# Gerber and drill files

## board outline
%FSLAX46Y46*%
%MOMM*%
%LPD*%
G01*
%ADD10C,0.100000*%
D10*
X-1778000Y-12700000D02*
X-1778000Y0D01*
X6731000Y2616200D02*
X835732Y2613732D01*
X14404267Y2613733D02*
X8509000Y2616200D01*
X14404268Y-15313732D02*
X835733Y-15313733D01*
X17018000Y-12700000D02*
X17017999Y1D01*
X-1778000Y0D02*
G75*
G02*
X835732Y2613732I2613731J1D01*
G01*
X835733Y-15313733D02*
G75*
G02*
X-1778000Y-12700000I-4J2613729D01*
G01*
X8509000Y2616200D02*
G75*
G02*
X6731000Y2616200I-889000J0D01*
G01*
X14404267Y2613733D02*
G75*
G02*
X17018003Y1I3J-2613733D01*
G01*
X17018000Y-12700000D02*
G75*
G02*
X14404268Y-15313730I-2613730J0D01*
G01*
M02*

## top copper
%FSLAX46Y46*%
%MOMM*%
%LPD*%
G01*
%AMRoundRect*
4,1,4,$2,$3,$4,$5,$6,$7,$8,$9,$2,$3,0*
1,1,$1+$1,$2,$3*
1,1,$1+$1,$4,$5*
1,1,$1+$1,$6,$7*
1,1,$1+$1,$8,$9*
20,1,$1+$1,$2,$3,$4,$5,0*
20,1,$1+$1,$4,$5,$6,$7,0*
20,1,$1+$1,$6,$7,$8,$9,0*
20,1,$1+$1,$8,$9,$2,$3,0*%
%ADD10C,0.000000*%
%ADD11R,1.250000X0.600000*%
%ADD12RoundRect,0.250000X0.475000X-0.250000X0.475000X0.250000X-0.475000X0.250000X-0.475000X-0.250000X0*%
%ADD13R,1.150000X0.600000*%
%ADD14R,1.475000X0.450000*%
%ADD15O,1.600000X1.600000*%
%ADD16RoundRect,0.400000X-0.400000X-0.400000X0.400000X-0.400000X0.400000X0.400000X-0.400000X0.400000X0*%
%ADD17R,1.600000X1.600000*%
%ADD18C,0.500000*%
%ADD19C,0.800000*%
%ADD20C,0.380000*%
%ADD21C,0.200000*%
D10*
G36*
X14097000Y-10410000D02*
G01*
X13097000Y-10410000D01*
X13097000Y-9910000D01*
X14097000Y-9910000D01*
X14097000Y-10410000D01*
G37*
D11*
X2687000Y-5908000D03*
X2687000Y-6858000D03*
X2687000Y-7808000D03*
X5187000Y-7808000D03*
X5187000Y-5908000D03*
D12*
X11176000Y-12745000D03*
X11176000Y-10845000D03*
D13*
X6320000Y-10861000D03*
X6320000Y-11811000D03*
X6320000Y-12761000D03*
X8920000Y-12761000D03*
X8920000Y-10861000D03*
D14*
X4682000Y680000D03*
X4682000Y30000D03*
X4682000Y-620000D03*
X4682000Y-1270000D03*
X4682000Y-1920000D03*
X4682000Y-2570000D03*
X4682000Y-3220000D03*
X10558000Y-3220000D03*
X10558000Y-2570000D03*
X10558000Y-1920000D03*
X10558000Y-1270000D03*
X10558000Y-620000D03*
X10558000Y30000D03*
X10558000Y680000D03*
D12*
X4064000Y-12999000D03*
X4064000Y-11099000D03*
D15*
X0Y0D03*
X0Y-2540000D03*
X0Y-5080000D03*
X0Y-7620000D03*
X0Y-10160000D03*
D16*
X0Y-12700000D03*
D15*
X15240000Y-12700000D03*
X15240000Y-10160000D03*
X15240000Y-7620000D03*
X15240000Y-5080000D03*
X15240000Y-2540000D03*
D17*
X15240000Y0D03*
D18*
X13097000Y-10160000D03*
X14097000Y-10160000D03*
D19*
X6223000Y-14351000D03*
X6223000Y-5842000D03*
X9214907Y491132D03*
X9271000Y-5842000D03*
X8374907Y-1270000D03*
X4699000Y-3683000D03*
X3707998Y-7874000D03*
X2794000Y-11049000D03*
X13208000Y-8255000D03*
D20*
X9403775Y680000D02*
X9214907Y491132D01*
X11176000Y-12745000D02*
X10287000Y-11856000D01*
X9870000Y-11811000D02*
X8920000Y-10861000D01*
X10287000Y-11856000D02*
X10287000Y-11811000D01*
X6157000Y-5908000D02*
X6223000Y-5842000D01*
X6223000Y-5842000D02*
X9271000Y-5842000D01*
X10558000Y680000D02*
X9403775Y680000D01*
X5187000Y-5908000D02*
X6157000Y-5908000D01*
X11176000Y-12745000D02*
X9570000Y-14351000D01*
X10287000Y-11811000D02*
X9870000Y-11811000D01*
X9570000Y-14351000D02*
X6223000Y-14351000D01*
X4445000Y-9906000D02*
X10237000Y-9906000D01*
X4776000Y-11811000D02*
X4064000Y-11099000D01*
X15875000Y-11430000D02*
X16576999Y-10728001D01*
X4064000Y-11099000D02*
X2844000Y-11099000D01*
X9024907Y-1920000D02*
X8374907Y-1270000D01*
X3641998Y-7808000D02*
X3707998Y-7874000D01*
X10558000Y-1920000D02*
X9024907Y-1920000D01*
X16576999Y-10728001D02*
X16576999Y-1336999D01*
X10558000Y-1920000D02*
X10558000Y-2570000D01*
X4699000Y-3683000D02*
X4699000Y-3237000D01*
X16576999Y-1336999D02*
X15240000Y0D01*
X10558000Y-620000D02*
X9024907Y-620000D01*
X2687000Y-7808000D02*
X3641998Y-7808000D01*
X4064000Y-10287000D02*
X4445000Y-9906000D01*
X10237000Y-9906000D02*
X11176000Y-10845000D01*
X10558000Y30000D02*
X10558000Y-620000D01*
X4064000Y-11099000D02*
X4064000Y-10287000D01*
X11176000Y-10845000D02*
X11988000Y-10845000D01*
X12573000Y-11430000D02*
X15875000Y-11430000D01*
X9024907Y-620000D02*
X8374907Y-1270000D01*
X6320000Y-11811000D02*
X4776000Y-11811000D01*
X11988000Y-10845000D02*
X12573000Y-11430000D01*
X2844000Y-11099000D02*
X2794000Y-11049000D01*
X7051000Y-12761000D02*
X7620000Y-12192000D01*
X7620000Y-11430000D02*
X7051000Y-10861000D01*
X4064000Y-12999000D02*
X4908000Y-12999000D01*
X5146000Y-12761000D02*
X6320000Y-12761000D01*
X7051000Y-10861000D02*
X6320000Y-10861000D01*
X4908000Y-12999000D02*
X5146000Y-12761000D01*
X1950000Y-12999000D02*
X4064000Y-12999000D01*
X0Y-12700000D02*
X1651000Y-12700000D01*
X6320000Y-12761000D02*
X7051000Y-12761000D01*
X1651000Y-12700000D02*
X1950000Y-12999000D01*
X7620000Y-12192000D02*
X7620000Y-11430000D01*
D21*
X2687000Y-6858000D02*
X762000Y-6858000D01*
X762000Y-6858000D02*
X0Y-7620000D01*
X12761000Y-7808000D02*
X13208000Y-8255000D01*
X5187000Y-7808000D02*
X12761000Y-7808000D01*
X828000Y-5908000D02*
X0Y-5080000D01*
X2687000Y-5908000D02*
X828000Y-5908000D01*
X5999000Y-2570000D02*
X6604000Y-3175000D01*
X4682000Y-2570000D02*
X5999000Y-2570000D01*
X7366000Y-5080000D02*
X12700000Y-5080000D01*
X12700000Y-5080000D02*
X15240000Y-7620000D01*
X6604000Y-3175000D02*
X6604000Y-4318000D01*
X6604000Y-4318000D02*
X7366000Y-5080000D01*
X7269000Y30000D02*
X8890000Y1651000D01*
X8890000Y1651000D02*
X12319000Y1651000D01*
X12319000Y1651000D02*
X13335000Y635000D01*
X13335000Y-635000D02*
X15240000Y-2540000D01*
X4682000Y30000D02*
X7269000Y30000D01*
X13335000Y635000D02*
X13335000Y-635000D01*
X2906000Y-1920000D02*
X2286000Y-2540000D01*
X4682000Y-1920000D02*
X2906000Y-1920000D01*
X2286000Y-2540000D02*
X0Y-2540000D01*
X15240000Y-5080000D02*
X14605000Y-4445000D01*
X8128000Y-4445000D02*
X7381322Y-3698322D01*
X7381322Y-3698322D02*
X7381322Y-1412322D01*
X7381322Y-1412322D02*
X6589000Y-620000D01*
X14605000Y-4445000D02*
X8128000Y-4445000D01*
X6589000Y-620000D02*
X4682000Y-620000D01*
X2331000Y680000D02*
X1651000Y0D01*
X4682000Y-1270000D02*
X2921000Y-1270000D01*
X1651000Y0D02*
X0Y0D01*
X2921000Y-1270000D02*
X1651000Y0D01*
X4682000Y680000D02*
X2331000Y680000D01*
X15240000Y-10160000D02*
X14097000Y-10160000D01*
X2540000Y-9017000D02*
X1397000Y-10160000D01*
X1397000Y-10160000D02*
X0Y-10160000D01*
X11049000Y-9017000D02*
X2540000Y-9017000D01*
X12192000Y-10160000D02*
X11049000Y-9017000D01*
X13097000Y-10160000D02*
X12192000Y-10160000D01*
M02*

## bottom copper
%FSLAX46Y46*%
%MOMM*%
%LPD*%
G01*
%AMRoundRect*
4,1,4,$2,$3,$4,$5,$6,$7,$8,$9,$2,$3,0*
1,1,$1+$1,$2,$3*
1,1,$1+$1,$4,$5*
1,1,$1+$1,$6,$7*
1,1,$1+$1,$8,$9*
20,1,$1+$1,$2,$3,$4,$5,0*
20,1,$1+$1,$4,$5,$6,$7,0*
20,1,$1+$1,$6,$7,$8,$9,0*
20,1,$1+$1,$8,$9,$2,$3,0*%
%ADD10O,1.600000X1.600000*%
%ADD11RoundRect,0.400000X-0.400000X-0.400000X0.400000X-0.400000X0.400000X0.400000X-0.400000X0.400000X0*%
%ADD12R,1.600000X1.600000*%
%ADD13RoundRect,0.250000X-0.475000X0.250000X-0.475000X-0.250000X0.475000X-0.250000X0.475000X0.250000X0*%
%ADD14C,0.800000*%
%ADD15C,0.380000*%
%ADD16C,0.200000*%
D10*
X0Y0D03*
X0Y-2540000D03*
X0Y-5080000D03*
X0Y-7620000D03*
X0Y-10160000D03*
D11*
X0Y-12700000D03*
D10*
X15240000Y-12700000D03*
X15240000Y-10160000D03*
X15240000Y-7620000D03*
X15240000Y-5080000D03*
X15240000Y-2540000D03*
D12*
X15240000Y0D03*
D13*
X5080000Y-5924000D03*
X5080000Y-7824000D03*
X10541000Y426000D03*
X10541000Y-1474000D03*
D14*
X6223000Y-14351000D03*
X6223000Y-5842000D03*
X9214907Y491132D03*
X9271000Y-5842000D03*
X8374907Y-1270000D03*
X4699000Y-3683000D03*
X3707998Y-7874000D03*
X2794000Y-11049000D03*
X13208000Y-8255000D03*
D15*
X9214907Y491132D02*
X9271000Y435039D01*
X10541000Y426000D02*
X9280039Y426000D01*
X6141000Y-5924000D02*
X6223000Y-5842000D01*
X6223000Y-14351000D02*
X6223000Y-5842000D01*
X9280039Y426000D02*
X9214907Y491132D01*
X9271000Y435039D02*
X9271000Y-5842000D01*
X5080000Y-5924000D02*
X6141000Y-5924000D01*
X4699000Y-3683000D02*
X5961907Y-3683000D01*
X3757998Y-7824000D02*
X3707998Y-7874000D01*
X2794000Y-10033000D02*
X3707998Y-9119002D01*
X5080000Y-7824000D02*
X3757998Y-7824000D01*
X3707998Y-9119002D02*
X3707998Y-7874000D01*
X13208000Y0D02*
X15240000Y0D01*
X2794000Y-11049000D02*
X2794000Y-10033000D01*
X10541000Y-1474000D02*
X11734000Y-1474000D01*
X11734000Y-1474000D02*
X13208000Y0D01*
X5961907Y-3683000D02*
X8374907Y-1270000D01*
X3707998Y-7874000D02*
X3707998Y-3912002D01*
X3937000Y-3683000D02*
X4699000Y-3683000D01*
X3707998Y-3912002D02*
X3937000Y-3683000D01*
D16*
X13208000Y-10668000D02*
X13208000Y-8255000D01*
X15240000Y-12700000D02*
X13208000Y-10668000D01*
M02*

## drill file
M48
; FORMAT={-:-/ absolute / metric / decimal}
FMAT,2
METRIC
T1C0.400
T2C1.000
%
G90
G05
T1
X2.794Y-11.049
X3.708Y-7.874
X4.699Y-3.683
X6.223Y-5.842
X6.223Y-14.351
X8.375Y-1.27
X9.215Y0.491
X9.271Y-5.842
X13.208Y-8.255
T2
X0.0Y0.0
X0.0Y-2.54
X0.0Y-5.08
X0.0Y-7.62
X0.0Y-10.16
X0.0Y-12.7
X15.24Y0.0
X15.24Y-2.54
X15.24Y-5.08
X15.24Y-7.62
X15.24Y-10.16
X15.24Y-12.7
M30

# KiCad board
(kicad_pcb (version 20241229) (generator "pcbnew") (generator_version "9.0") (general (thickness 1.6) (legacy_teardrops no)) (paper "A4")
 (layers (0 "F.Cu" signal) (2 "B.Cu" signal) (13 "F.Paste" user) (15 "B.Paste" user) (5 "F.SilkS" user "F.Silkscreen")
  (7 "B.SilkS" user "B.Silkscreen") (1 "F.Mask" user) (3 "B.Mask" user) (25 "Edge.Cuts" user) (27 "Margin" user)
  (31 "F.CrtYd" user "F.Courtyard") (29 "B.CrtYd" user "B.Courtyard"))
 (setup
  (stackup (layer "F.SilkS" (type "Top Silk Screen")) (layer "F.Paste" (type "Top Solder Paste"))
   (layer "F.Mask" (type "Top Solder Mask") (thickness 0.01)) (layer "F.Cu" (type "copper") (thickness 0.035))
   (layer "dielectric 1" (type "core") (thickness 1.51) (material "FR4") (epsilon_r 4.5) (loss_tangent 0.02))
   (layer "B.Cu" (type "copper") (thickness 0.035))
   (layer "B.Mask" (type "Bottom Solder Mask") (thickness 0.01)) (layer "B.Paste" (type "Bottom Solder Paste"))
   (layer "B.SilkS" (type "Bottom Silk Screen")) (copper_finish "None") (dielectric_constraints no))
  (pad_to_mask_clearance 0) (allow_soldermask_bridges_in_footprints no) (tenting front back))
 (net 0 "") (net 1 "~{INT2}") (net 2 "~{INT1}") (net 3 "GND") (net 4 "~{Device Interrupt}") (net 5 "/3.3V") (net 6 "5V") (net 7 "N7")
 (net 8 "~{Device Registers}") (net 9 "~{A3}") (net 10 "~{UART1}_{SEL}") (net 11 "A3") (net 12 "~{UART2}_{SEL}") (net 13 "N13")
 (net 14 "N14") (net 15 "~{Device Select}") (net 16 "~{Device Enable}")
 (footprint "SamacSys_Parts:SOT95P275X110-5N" (layer "F.Cu") (at 3.937 6.858)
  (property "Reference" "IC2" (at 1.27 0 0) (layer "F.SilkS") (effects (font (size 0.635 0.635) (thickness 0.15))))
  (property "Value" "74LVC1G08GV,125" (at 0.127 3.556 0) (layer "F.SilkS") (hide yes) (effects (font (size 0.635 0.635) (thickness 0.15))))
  (pad "1" smd rect (at -1.25 -0.95 90) (size 0.6 1.25) (layers "F.Cu" "F.Mask" "F.Paste") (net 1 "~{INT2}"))
  (pad "2" smd rect (at -1.25 0 90) (size 0.6 1.25) (layers "F.Cu" "F.Mask" "F.Paste") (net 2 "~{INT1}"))
  (pad "3" smd rect (at -1.25 0.95 90) (size 0.6 1.25) (layers "F.Cu" "F.Mask" "F.Paste") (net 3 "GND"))
  (pad "4" smd rect (at 1.25 0.95 90) (size 0.6 1.25) (layers "F.Cu" "F.Mask" "F.Paste") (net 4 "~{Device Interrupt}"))
  (pad "5" smd rect (at 1.25 -0.95 90) (size 0.6 1.25) (layers "F.Cu" "F.Mask" "F.Paste") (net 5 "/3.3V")))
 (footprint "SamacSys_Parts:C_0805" (layer "F.Cu") (at 11.176 11.811)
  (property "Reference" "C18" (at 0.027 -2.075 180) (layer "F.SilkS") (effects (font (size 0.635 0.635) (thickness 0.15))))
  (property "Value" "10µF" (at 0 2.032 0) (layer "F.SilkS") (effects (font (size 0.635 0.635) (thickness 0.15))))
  (pad "1" smd roundrect (at 0 0.934 90) (size 1 1.45) (layers "F.Cu" "F.Mask" "F.Paste") (roundrect_rratio 0.25) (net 5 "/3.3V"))
  (pad "2" smd roundrect (at 0 -0.966 90) (size 1 1.45) (layers "F.Cu" "F.Mask" "F.Paste") (roundrect_rratio 0.25) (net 3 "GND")))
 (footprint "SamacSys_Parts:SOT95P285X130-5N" (layer "F.Cu") (at 7.62 11.811)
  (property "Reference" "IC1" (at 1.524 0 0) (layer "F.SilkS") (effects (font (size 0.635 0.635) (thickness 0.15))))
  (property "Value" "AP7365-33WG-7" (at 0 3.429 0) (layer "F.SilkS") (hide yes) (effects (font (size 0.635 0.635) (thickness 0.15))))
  (pad "1" smd rect (at -1.3 -0.95 90) (size 0.6 1.15) (layers "F.Cu" "F.Mask" "F.Paste") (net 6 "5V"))
  (pad "2" smd rect (at -1.3 0 90) (size 0.6 1.15) (layers "F.Cu" "F.Mask" "F.Paste") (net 3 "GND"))
  (pad "3" smd rect (at -1.3 0.95 90) (size 0.6 1.15) (layers "F.Cu" "F.Mask" "F.Paste") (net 6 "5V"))
  (pad "4" smd rect (at 1.3 0.95 90) (size 0.6 1.15) (layers "F.Cu" "F.Mask" "F.Paste") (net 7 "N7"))
  (pad "5" smd rect (at 1.3 -0.95 90) (size 0.6 1.15) (layers "F.Cu" "F.Mask" "F.Paste") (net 5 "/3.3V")))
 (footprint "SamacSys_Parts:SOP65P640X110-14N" (layer "F.Cu") (at 7.62 1.27)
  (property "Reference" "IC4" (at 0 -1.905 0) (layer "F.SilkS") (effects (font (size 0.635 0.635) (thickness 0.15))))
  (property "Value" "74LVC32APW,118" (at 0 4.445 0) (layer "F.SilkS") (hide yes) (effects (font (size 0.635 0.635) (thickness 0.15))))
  (pad "1" smd rect (at -2.938 -1.95 90) (size 0.45 1.475) (layers "F.Cu" "F.Mask" "F.Paste") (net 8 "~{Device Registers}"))
  (pad "2" smd rect (at -2.938 -1.3 90) (size 0.45 1.475) (layers "F.Cu" "F.Mask" "F.Paste") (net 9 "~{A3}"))
  (pad "3" smd rect (at -2.938 -0.65 90) (size 0.45 1.475) (layers "F.Cu" "F.Mask" "F.Paste") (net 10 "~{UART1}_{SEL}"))
  (pad "4" smd rect (at -2.938 0 90) (size 0.45 1.475) (layers "F.Cu" "F.Mask" "F.Paste") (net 8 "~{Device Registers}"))
  (pad "5" smd rect (at -2.938 0.65 90) (size 0.45 1.475) (layers "F.Cu" "F.Mask" "F.Paste") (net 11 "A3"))
  (pad "6" smd rect (at -2.938 1.3 90) (size 0.45 1.475) (layers "F.Cu" "F.Mask" "F.Paste") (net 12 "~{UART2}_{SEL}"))
  (pad "7" smd rect (at -2.938 1.95 90) (size 0.45 1.475) (layers "F.Cu" "F.Mask" "F.Paste") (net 3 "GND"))
  (pad "8" smd rect (at 2.938 1.95 90) (size 0.45 1.475) (layers "F.Cu" "F.Mask" "F.Paste") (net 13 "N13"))
  (pad "9" smd rect (at 2.938 1.3 90) (size 0.45 1.475) (layers "F.Cu" "F.Mask" "F.Paste") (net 3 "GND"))
  (pad "10" smd rect (at 2.938 0.65 90) (size 0.45 1.475) (layers "F.Cu" "F.Mask" "F.Paste") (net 3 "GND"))
  (pad "11" smd rect (at 2.938 0 90) (size 0.45 1.475) (layers "F.Cu" "F.Mask" "F.Paste") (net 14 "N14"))
  (pad "12" smd rect (at 2.938 -0.65 90) (size 0.45 1.475) (layers "F.Cu" "F.Mask" "F.Paste") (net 3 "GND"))
  (pad "13" smd rect (at 2.938 -1.3 90) (size 0.45 1.475) (layers "F.Cu" "F.Mask" "F.Paste") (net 3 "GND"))
  (pad "14" smd rect (at 2.938 -1.95 90) (size 0.45 1.475) (layers "F.Cu" "F.Mask" "F.Paste") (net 5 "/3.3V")))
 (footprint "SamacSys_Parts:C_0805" (layer "F.Cu") (at 4.064 12.065)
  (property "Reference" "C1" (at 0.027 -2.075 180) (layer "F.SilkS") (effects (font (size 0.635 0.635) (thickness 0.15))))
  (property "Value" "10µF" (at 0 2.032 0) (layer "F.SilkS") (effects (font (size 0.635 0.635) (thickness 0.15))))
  (pad "1" smd roundrect (at 0 0.934 90) (size 1 1.45) (layers "F.Cu" "F.Mask" "F.Paste") (roundrect_rratio 0.25) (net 6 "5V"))
  (pad "2" smd roundrect (at 0 -0.966 90) (size 1 1.45) (layers "F.Cu" "F.Mask" "F.Paste") (roundrect_rratio 0.25) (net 3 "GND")))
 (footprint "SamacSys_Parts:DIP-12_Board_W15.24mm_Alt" (layer "F.Cu") (at 0 0)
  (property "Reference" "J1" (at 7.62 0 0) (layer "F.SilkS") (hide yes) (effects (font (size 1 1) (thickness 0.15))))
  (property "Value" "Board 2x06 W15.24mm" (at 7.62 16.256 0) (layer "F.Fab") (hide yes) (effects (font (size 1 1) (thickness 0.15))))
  (fp_line (start -1.778 12.7) (end -1.778 0) (stroke (width 0.1) (type solid)) (layer "Edge.Cuts"))
  (fp_line (start 6.731 -2.6162) (end 0.835732 -2.613732) (stroke (width 0.1) (type solid)) (layer "Edge.Cuts"))
  (fp_line (start 14.404267 -2.613733) (end 8.509 -2.6162) (stroke (width 0.1) (type solid)) (layer "Edge.Cuts"))
  (fp_line (start 14.404268 15.313732) (end 0.835733 15.313733) (stroke (width 0.1) (type solid)) (layer "Edge.Cuts"))
  (fp_line (start 17.018 12.7) (end 17.017999 -0.000001) (stroke (width 0.1) (type solid)) (layer "Edge.Cuts"))
  (fp_arc (start -1.778 0) (mid -1.012456 -1.848188) (end 0.835732 -2.613732) (stroke (width 0.1) (type solid)) (layer "Edge.Cuts"))
  (fp_arc (start 0.835733 15.313733) (mid -1.012457 14.548189) (end -1.778 12.7) (stroke (width 0.1) (type solid)) (layer "Edge.Cuts"))
  (fp_arc (start 8.509 -2.6162) (mid 7.62 -1.7272) (end 6.731 -2.6162) (stroke (width 0.1) (type default)) (layer "Edge.Cuts"))
  (fp_arc (start 14.404267 -2.613733) (mid 16.252455 -1.848189) (end 17.017999 -0.000001) (stroke (width 0.1) (type solid))
   (layer "Edge.Cuts"))
  (fp_arc (start 17.018 12.7) (mid 16.252456 14.548187) (end 14.404268 15.313732) (stroke (width 0.1) (type solid)) (layer "Edge.Cuts"))
  (pad "1" thru_hole oval (at 0 0 180) (size 1.6 1.6) (drill 1) (layers "*.Cu" "*.Mask") (remove_unused_layers no)
   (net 8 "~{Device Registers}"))
  (pad "2" thru_hole oval (at 0 2.54) (size 1.6 1.6) (drill 1) (layers "*.Cu" "*.Mask") (remove_unused_layers no) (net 11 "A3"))
  (pad "3" thru_hole oval (at 0 5.08) (size 1.6 1.6) (drill 1) (layers "*.Cu" "*.Mask") (remove_unused_layers no) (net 1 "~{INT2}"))
  (pad "4" thru_hole oval (at 0 7.62 180) (size 1.6 1.6) (drill 1) (layers "*.Cu" "*.Mask") (remove_unused_layers no) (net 2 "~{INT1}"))
  (pad "5" thru_hole oval (at 0 10.16) (size 1.6 1.6) (drill 1) (layers "*.Cu" "*.Mask") (remove_unused_layers no)
   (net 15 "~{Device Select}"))
  (pad "6" thru_hole roundrect (at 0 12.7) (size 1.6 1.6) (drill 1) (layers "*.Cu" "*.Mask") (remove_unused_layers no)
   (roundrect_rratio 0.25) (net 6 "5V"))
  (pad "7" thru_hole oval (at 15.24 12.7 180) (size 1.6 1.6) (drill 1) (layers "*.Cu" "*.Mask") (remove_unused_layers no)
   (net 4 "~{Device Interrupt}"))
  (pad "8" thru_hole oval (at 15.24 10.16 180) (size 1.6 1.6) (drill 1) (layers "*.Cu" "*.Mask") (remove_unused_layers no)
   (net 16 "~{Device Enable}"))
  (pad "9" thru_hole oval (at 15.24 7.62 180) (size 1.6 1.6) (drill 1) (layers "*.Cu" "*.Mask") (remove_unused_layers no)
   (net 12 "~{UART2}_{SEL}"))
  (pad "10" thru_hole oval (at 15.24 5.08) (size 1.6 1.6) (drill 1) (layers "*.Cu" "*.Mask") (remove_unused_layers no)
   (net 10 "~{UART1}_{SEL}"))
  (pad "11" thru_hole oval (at 15.24 2.54) (size 1.6 1.6) (drill 1) (layers "*.Cu" "*.Mask") (remove_unused_layers no) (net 9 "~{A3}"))
  (pad "12" thru_hole rect (at 15.24 0) (size 1.6 1.6) (drill 1) (layers "*.Cu" "*.Mask") (remove_unused_layers no) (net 3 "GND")))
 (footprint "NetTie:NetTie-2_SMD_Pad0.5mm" (layer "F.Cu") (at 13.597 10.16)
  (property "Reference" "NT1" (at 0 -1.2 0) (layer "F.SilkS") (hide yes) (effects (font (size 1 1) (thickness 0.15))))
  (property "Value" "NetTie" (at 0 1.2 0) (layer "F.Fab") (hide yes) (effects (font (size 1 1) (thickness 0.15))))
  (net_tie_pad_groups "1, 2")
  (fp_poly (pts (xy -0.5 -0.25) (xy 0.5 -0.25) (xy 0.5 0.25) (xy -0.5 0.25)) (stroke (width 0) (type solid)) (fill yes) (layer "F.Cu"))
  (pad "1" smd circle (at -0.5 0) (size 0.5 0.5) (layers "F.Cu") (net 15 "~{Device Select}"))
  (pad "2" smd circle (at 0.5 0) (size 0.5 0.5) (layers "F.Cu") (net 16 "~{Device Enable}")))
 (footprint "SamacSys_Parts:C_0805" (layer "B.Cu") (at 5.08 6.858)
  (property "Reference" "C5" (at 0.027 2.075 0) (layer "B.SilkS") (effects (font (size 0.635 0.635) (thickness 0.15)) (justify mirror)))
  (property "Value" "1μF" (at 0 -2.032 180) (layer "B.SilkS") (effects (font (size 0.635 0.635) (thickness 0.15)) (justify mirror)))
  (pad "1" smd roundrect (at 0 -0.934 270) (size 1 1.45) (layers "B.Cu" "B.Mask" "B.Paste") (roundrect_rratio 0.25) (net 5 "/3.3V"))
  (pad "2" smd roundrect (at 0 0.966 270) (size 1 1.45) (layers "B.Cu" "B.Mask" "B.Paste") (roundrect_rratio 0.25) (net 3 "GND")))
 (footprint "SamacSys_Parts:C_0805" (layer "B.Cu") (at 10.541 0.508)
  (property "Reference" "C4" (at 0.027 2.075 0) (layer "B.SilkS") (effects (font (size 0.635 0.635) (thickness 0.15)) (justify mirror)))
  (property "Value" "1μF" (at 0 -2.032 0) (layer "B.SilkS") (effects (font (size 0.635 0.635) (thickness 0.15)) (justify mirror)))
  (pad "1" smd roundrect (at 0 -0.934 270) (size 1 1.45) (layers "B.Cu" "B.Mask" "B.Paste") (roundrect_rratio 0.25) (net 5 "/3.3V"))
  (pad "2" smd roundrect (at 0 0.966 270) (size 1 1.45) (layers "B.Cu" "B.Mask" "B.Paste") (roundrect_rratio 0.25) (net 3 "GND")))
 (segment (start 9.403775 -0.68) (end 9.214907 -0.491132) (width 0.38) (layer "F.Cu") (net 5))
 (segment (start 11.176 12.745) (end 10.287 11.856) (width 0.38) (layer "F.Cu") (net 5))
 (segment (start 9.87 11.811) (end 8.92 10.861) (width 0.38) (layer "F.Cu") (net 5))
 (segment (start 10.287 11.856) (end 10.287 11.811) (width 0.38) (layer "F.Cu") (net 5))
 (segment (start 6.157 5.908) (end 6.223 5.842) (width 0.38) (layer "F.Cu") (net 5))
 (segment (start 6.223 5.842) (end 9.271 5.842) (width 0.38) (layer "F.Cu") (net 5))
 (segment (start 10.558 -0.68) (end 9.403775 -0.68) (width 0.38) (layer "F.Cu") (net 5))
 (segment (start 5.187 5.908) (end 6.157 5.908) (width 0.38) (layer "F.Cu") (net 5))
 (segment (start 11.176 12.745) (end 9.57 14.351) (width 0.38) (layer "F.Cu") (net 5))
 (segment (start 10.287 11.811) (end 9.87 11.811) (width 0.38) (layer "F.Cu") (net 5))
 (segment (start 9.57 14.351) (end 6.223 14.351) (width 0.38) (layer "F.Cu") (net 5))
 (via (at 6.223 14.351) (size 0.8) (drill 0.4) (layers "F.Cu" "B.Cu") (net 5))
 (via (at 6.223 5.842) (size 0.8) (drill 0.4) (layers "F.Cu" "B.Cu") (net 5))
 (via (at 9.214907 -0.491132) (size 0.8) (drill 0.4) (layers "F.Cu" "B.Cu") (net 5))
 (via (at 9.271 5.842) (size 0.8) (drill 0.4) (layers "F.Cu" "B.Cu") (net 5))
 (segment (start 9.214907 -0.491132) (end 9.271 -0.435039) (width 0.38) (layer "B.Cu") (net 5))
 (segment (start 10.541 -0.426) (end 9.280039 -0.426) (width 0.38) (layer "B.Cu") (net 5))
 (segment (start 6.141 5.924) (end 6.223 5.842) (width 0.38) (layer "B.Cu") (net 5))
 (segment (start 6.223 14.351) (end 6.223 5.842) (width 0.38) (layer "B.Cu") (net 5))
 (segment (start 9.280039 -0.426) (end 9.214907 -0.491132) (width 0.38) (layer "B.Cu") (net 5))
 (segment (start 9.271 -0.435039) (end 9.271 5.842) (width 0.38) (layer "B.Cu") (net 5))
 (segment (start 5.08 5.924) (end 6.141 5.924) (width 0.38) (layer "B.Cu") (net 5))
 (segment (start 4.445 9.906) (end 10.237 9.906) (width 0.38) (layer "F.Cu") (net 3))
 (segment (start 4.776 11.811) (end 4.064 11.099) (width 0.38) (layer "F.Cu") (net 3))
 (segment (start 15.875 11.43) (end 16.576999 10.728001) (width 0.38) (layer "F.Cu") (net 3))
 (segment (start 4.064 11.099) (end 2.844 11.099) (width 0.38) (layer "F.Cu") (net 3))
 (segment (start 9.024907 1.92) (end 8.374907 1.27) (width 0.38) (layer "F.Cu") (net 3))
 (segment (start 3.641998 7.808) (end 3.707998 7.874) (width 0.38) (layer "F.Cu") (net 3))
 (segment (start 10.558 1.92) (end 9.024907 1.92) (width 0.38) (layer "F.Cu") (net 3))
 (segment (start 16.576999 10.728001) (end 16.576999 1.336999) (width 0.38) (layer "F.Cu") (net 3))
 (segment (start 10.558 1.92) (end 10.558 2.57) (width 0.38) (layer "F.Cu") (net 3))
 (segment (start 4.699 3.683) (end 4.699 3.237) (width 0.38) (layer "F.Cu") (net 3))
 (segment (start 16.576999 1.336999) (end 15.24 0) (width 0.38) (layer "F.Cu") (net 3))
 (segment (start 10.558 0.62) (end 9.024907 0.62) (width 0.38) (layer "F.Cu") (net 3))
 (segment (start 2.687 7.808) (end 3.641998 7.808) (width 0.38) (layer "F.Cu") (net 3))
 (segment (start 4.064 10.287) (end 4.445 9.906) (width 0.38) (layer "F.Cu") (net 3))
 (segment (start 10.237 9.906) (end 11.176 10.845) (width 0.38) (layer "F.Cu") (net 3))
 (segment (start 10.558 -0.03) (end 10.558 0.62) (width 0.38) (layer "F.Cu") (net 3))
 (segment (start 4.064 11.099) (end 4.064 10.287) (width 0.38) (layer "F.Cu") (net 3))
 (segment (start 11.176 10.845) (end 11.988 10.845) (width 0.38) (layer "F.Cu") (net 3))
 (segment (start 12.573 11.43) (end 15.875 11.43) (width 0.38) (layer "F.Cu") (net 3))
 (segment (start 9.024907 0.62) (end 8.374907 1.27) (width 0.38) (layer "F.Cu") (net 3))
 (segment (start 6.32 11.811) (end 4.776 11.811) (width 0.38) (layer "F.Cu") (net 3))
 (segment (start 11.988 10.845) (end 12.573 11.43) (width 0.38) (layer "F.Cu") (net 3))
 (segment (start 2.844 11.099) (end 2.794 11.049) (width 0.38) (layer "F.Cu") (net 3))
 (via (at 8.374907 1.27) (size 0.8) (drill 0.4) (layers "F.Cu" "B.Cu") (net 3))
 (via (at 4.699 3.683) (size 0.8) (drill 0.4) (layers "F.Cu" "B.Cu") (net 3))
 (via (at 3.707998 7.874) (size 0.8) (drill 0.4) (layers "F.Cu" "B.Cu") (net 3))
 (via (at 2.794 11.049) (size 0.8) (drill 0.4) (layers "F.Cu" "B.Cu") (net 3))
 (segment (start 4.699 3.683) (end 5.961907 3.683) (width 0.38) (layer "B.Cu") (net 3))
 (segment (start 3.757998 7.824) (end 3.707998 7.874) (width 0.38) (layer "B.Cu") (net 3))
 (segment (start 2.794 10.033) (end 3.707998 9.119002) (width 0.38) (layer "B.Cu") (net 3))
 (segment (start 5.08 7.824) (end 3.757998 7.824) (width 0.38) (layer "B.Cu") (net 3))
 (segment (start 3.707998 9.119002) (end 3.707998 7.874) (width 0.38) (layer "B.Cu") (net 3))
 (segment (start 13.208 0) (end 15.24 0) (width 0.38) (layer "B.Cu") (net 3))
 (segment (start 2.794 11.049) (end 2.794 10.033) (width 0.38) (layer "B.Cu") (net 3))
 (segment (start 10.541 1.474) (end 11.734 1.474) (width 0.38) (layer "B.Cu") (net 3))
 (segment (start 11.734 1.474) (end 13.208 0) (width 0.38) (layer "B.Cu") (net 3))
 (segment (start 5.961907 3.683) (end 8.374907 1.27) (width 0.38) (layer "B.Cu") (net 3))
 (segment (start 3.707998 7.874) (end 3.707998 3.912002) (width 0.38) (layer "B.Cu") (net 3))
 (segment (start 3.937 3.683) (end 4.699 3.683) (width 0.38) (layer "B.Cu") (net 3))
 (segment (start 3.707998 3.912002) (end 3.937 3.683) (width 0.38) (layer "B.Cu") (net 3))
 (segment (start 7.051 12.761) (end 7.62 12.192) (width 0.38) (layer "F.Cu") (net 6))
 (segment (start 7.62 11.43) (end 7.051 10.861) (width 0.38) (layer "F.Cu") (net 6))
 (segment (start 4.064 12.999) (end 4.908 12.999) (width 0.38) (layer "F.Cu") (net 6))
 (segment (start 5.146 12.761) (end 6.32 12.761) (width 0.38) (layer "F.Cu") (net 6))
 (segment (start 7.051 10.861) (end 6.32 10.861) (width 0.38) (layer "F.Cu") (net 6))
 (segment (start 4.908 12.999) (end 5.146 12.761) (width 0.38) (layer "F.Cu") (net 6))
 (segment (start 1.95 12.999) (end 4.064 12.999) (width 0.38) (layer "F.Cu") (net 6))
 (segment (start 0 12.7) (end 1.651 12.7) (width 0.38) (layer "F.Cu") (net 6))
 (segment (start 6.32 12.761) (end 7.051 12.761) (width 0.38) (layer "F.Cu") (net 6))
 (segment (start 1.651 12.7) (end 1.95 12.999) (width 0.38) (layer "F.Cu") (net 6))
 (segment (start 7.62 12.192) (end 7.62 11.43) (width 0.38) (layer "F.Cu") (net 6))
 (segment (start 2.687 6.858) (end 0.762 6.858) (width 0.2) (layer "F.Cu") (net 2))
 (segment (start 0.762 6.858) (end 0 7.62) (width 0.2) (layer "F.Cu") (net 2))
 (segment (start 12.761 7.808) (end 13.208 8.255) (width 0.2) (layer "F.Cu") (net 4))
 (segment (start 5.187 7.808) (end 12.761 7.808) (width 0.2) (layer "F.Cu") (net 4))
 (via (at 13.208 8.255) (size 0.8) (drill 0.4) (layers "F.Cu" "B.Cu") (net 4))
 (segment (start 13.208 10.668) (end 13.208 8.255) (width 0.2) (layer "B.Cu") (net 4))
 (segment (start 15.24 12.7) (end 13.208 10.668) (width 0.2) (layer "B.Cu") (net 4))
 (segment (start 0.828 5.908) (end 0 5.08) (width 0.2) (layer "F.Cu") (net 1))
 (segment (start 2.687 5.908) (end 0.828 5.908) (width 0.2) (layer "F.Cu") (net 1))
 (segment (start 5.999 2.57) (end 6.604 3.175) (width 0.2) (layer "F.Cu") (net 12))
 (segment (start 4.682 2.57) (end 5.999 2.57) (width 0.2) (layer "F.Cu") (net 12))
 (segment (start 7.366 5.08) (end 12.7 5.08) (width 0.2) (layer "F.Cu") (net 12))
 (segment (start 12.7 5.08) (end 15.24 7.62) (width 0.2) (layer "F.Cu") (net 12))
 (segment (start 6.604 3.175) (end 6.604 4.318) (width 0.2) (layer "F.Cu") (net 12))
 (segment (start 6.604 4.318) (end 7.366 5.08) (width 0.2) (layer "F.Cu") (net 12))
 (segment (start 7.269 -0.03) (end 8.89 -1.651) (width 0.2) (layer "F.Cu") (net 9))
 (segment (start 8.89 -1.651) (end 12.319 -1.651) (width 0.2) (layer "F.Cu") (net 9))
 (segment (start 12.319 -1.651) (end 13.335 -0.635) (width 0.2) (layer "F.Cu") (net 9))
 (segment (start 13.335 0.635) (end 15.24 2.54) (width 0.2) (layer "F.Cu") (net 9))
 (segment (start 4.682 -0.03) (end 7.269 -0.03) (width 0.2) (layer "F.Cu") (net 9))
 (segment (start 13.335 -0.635) (end 13.335 0.635) (width 0.2) (layer "F.Cu") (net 9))
 (segment (start 2.906 1.92) (end 2.286 2.54) (width 0.2) (layer "F.Cu") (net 11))
 (segment (start 4.682 1.92) (end 2.906 1.92) (width 0.2) (layer "F.Cu") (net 11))
 (segment (start 2.286 2.54) (end 0 2.54) (width 0.2) (layer "F.Cu") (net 11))
 (segment (start 15.24 5.08) (end 14.605 4.445) (width 0.2) (layer "F.Cu") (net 10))
 (segment (start 8.128 4.445) (end 7.381322 3.698322) (width 0.2) (layer "F.Cu") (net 10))
 (segment (start 7.381322 3.698322) (end 7.381322 1.412322) (width 0.2) (layer "F.Cu") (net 10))
 (segment (start 7.381322 1.412322) (end 6.589 0.62) (width 0.2) (layer "F.Cu") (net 10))
 (segment (start 14.605 4.445) (end 8.128 4.445) (width 0.2) (layer "F.Cu") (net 10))
 (segment (start 6.589 0.62) (end 4.682 0.62) (width 0.2) (layer "F.Cu") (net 10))
 (segment (start 2.331 -0.68) (end 1.651 0) (width 0.2) (layer "F.Cu") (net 8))
 (segment (start 4.682 1.27) (end 2.921 1.27) (width 0.2) (layer "F.Cu") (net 8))
 (segment (start 1.651 0) (end 0 0) (width 0.2) (layer "F.Cu") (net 8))
 (segment (start 2.921 1.27) (end 1.651 0) (width 0.2) (layer "F.Cu") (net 8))
 (segment (start 4.682 -0.68) (end 2.331 -0.68) (width 0.2) (layer "F.Cu") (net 8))
 (segment (start 15.24 10.16) (end 14.097 10.16) (width 0.2) (layer "F.Cu") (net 16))
 (segment (start 2.54 9.017) (end 1.397 10.16) (width 0.2) (layer "F.Cu") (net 15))
 (segment (start 1.397 10.16) (end 0 10.16) (width 0.2) (layer "F.Cu") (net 15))
 (segment (start 11.049 9.017) (end 2.54 9.017) (width 0.2) (layer "F.Cu") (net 15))
 (segment (start 12.192 10.16) (end 11.049 9.017) (width 0.2) (layer "F.Cu") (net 15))
 (segment (start 13.097 10.16) (end 12.192 10.16) (width 0.2) (layer "F.Cu") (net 15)))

